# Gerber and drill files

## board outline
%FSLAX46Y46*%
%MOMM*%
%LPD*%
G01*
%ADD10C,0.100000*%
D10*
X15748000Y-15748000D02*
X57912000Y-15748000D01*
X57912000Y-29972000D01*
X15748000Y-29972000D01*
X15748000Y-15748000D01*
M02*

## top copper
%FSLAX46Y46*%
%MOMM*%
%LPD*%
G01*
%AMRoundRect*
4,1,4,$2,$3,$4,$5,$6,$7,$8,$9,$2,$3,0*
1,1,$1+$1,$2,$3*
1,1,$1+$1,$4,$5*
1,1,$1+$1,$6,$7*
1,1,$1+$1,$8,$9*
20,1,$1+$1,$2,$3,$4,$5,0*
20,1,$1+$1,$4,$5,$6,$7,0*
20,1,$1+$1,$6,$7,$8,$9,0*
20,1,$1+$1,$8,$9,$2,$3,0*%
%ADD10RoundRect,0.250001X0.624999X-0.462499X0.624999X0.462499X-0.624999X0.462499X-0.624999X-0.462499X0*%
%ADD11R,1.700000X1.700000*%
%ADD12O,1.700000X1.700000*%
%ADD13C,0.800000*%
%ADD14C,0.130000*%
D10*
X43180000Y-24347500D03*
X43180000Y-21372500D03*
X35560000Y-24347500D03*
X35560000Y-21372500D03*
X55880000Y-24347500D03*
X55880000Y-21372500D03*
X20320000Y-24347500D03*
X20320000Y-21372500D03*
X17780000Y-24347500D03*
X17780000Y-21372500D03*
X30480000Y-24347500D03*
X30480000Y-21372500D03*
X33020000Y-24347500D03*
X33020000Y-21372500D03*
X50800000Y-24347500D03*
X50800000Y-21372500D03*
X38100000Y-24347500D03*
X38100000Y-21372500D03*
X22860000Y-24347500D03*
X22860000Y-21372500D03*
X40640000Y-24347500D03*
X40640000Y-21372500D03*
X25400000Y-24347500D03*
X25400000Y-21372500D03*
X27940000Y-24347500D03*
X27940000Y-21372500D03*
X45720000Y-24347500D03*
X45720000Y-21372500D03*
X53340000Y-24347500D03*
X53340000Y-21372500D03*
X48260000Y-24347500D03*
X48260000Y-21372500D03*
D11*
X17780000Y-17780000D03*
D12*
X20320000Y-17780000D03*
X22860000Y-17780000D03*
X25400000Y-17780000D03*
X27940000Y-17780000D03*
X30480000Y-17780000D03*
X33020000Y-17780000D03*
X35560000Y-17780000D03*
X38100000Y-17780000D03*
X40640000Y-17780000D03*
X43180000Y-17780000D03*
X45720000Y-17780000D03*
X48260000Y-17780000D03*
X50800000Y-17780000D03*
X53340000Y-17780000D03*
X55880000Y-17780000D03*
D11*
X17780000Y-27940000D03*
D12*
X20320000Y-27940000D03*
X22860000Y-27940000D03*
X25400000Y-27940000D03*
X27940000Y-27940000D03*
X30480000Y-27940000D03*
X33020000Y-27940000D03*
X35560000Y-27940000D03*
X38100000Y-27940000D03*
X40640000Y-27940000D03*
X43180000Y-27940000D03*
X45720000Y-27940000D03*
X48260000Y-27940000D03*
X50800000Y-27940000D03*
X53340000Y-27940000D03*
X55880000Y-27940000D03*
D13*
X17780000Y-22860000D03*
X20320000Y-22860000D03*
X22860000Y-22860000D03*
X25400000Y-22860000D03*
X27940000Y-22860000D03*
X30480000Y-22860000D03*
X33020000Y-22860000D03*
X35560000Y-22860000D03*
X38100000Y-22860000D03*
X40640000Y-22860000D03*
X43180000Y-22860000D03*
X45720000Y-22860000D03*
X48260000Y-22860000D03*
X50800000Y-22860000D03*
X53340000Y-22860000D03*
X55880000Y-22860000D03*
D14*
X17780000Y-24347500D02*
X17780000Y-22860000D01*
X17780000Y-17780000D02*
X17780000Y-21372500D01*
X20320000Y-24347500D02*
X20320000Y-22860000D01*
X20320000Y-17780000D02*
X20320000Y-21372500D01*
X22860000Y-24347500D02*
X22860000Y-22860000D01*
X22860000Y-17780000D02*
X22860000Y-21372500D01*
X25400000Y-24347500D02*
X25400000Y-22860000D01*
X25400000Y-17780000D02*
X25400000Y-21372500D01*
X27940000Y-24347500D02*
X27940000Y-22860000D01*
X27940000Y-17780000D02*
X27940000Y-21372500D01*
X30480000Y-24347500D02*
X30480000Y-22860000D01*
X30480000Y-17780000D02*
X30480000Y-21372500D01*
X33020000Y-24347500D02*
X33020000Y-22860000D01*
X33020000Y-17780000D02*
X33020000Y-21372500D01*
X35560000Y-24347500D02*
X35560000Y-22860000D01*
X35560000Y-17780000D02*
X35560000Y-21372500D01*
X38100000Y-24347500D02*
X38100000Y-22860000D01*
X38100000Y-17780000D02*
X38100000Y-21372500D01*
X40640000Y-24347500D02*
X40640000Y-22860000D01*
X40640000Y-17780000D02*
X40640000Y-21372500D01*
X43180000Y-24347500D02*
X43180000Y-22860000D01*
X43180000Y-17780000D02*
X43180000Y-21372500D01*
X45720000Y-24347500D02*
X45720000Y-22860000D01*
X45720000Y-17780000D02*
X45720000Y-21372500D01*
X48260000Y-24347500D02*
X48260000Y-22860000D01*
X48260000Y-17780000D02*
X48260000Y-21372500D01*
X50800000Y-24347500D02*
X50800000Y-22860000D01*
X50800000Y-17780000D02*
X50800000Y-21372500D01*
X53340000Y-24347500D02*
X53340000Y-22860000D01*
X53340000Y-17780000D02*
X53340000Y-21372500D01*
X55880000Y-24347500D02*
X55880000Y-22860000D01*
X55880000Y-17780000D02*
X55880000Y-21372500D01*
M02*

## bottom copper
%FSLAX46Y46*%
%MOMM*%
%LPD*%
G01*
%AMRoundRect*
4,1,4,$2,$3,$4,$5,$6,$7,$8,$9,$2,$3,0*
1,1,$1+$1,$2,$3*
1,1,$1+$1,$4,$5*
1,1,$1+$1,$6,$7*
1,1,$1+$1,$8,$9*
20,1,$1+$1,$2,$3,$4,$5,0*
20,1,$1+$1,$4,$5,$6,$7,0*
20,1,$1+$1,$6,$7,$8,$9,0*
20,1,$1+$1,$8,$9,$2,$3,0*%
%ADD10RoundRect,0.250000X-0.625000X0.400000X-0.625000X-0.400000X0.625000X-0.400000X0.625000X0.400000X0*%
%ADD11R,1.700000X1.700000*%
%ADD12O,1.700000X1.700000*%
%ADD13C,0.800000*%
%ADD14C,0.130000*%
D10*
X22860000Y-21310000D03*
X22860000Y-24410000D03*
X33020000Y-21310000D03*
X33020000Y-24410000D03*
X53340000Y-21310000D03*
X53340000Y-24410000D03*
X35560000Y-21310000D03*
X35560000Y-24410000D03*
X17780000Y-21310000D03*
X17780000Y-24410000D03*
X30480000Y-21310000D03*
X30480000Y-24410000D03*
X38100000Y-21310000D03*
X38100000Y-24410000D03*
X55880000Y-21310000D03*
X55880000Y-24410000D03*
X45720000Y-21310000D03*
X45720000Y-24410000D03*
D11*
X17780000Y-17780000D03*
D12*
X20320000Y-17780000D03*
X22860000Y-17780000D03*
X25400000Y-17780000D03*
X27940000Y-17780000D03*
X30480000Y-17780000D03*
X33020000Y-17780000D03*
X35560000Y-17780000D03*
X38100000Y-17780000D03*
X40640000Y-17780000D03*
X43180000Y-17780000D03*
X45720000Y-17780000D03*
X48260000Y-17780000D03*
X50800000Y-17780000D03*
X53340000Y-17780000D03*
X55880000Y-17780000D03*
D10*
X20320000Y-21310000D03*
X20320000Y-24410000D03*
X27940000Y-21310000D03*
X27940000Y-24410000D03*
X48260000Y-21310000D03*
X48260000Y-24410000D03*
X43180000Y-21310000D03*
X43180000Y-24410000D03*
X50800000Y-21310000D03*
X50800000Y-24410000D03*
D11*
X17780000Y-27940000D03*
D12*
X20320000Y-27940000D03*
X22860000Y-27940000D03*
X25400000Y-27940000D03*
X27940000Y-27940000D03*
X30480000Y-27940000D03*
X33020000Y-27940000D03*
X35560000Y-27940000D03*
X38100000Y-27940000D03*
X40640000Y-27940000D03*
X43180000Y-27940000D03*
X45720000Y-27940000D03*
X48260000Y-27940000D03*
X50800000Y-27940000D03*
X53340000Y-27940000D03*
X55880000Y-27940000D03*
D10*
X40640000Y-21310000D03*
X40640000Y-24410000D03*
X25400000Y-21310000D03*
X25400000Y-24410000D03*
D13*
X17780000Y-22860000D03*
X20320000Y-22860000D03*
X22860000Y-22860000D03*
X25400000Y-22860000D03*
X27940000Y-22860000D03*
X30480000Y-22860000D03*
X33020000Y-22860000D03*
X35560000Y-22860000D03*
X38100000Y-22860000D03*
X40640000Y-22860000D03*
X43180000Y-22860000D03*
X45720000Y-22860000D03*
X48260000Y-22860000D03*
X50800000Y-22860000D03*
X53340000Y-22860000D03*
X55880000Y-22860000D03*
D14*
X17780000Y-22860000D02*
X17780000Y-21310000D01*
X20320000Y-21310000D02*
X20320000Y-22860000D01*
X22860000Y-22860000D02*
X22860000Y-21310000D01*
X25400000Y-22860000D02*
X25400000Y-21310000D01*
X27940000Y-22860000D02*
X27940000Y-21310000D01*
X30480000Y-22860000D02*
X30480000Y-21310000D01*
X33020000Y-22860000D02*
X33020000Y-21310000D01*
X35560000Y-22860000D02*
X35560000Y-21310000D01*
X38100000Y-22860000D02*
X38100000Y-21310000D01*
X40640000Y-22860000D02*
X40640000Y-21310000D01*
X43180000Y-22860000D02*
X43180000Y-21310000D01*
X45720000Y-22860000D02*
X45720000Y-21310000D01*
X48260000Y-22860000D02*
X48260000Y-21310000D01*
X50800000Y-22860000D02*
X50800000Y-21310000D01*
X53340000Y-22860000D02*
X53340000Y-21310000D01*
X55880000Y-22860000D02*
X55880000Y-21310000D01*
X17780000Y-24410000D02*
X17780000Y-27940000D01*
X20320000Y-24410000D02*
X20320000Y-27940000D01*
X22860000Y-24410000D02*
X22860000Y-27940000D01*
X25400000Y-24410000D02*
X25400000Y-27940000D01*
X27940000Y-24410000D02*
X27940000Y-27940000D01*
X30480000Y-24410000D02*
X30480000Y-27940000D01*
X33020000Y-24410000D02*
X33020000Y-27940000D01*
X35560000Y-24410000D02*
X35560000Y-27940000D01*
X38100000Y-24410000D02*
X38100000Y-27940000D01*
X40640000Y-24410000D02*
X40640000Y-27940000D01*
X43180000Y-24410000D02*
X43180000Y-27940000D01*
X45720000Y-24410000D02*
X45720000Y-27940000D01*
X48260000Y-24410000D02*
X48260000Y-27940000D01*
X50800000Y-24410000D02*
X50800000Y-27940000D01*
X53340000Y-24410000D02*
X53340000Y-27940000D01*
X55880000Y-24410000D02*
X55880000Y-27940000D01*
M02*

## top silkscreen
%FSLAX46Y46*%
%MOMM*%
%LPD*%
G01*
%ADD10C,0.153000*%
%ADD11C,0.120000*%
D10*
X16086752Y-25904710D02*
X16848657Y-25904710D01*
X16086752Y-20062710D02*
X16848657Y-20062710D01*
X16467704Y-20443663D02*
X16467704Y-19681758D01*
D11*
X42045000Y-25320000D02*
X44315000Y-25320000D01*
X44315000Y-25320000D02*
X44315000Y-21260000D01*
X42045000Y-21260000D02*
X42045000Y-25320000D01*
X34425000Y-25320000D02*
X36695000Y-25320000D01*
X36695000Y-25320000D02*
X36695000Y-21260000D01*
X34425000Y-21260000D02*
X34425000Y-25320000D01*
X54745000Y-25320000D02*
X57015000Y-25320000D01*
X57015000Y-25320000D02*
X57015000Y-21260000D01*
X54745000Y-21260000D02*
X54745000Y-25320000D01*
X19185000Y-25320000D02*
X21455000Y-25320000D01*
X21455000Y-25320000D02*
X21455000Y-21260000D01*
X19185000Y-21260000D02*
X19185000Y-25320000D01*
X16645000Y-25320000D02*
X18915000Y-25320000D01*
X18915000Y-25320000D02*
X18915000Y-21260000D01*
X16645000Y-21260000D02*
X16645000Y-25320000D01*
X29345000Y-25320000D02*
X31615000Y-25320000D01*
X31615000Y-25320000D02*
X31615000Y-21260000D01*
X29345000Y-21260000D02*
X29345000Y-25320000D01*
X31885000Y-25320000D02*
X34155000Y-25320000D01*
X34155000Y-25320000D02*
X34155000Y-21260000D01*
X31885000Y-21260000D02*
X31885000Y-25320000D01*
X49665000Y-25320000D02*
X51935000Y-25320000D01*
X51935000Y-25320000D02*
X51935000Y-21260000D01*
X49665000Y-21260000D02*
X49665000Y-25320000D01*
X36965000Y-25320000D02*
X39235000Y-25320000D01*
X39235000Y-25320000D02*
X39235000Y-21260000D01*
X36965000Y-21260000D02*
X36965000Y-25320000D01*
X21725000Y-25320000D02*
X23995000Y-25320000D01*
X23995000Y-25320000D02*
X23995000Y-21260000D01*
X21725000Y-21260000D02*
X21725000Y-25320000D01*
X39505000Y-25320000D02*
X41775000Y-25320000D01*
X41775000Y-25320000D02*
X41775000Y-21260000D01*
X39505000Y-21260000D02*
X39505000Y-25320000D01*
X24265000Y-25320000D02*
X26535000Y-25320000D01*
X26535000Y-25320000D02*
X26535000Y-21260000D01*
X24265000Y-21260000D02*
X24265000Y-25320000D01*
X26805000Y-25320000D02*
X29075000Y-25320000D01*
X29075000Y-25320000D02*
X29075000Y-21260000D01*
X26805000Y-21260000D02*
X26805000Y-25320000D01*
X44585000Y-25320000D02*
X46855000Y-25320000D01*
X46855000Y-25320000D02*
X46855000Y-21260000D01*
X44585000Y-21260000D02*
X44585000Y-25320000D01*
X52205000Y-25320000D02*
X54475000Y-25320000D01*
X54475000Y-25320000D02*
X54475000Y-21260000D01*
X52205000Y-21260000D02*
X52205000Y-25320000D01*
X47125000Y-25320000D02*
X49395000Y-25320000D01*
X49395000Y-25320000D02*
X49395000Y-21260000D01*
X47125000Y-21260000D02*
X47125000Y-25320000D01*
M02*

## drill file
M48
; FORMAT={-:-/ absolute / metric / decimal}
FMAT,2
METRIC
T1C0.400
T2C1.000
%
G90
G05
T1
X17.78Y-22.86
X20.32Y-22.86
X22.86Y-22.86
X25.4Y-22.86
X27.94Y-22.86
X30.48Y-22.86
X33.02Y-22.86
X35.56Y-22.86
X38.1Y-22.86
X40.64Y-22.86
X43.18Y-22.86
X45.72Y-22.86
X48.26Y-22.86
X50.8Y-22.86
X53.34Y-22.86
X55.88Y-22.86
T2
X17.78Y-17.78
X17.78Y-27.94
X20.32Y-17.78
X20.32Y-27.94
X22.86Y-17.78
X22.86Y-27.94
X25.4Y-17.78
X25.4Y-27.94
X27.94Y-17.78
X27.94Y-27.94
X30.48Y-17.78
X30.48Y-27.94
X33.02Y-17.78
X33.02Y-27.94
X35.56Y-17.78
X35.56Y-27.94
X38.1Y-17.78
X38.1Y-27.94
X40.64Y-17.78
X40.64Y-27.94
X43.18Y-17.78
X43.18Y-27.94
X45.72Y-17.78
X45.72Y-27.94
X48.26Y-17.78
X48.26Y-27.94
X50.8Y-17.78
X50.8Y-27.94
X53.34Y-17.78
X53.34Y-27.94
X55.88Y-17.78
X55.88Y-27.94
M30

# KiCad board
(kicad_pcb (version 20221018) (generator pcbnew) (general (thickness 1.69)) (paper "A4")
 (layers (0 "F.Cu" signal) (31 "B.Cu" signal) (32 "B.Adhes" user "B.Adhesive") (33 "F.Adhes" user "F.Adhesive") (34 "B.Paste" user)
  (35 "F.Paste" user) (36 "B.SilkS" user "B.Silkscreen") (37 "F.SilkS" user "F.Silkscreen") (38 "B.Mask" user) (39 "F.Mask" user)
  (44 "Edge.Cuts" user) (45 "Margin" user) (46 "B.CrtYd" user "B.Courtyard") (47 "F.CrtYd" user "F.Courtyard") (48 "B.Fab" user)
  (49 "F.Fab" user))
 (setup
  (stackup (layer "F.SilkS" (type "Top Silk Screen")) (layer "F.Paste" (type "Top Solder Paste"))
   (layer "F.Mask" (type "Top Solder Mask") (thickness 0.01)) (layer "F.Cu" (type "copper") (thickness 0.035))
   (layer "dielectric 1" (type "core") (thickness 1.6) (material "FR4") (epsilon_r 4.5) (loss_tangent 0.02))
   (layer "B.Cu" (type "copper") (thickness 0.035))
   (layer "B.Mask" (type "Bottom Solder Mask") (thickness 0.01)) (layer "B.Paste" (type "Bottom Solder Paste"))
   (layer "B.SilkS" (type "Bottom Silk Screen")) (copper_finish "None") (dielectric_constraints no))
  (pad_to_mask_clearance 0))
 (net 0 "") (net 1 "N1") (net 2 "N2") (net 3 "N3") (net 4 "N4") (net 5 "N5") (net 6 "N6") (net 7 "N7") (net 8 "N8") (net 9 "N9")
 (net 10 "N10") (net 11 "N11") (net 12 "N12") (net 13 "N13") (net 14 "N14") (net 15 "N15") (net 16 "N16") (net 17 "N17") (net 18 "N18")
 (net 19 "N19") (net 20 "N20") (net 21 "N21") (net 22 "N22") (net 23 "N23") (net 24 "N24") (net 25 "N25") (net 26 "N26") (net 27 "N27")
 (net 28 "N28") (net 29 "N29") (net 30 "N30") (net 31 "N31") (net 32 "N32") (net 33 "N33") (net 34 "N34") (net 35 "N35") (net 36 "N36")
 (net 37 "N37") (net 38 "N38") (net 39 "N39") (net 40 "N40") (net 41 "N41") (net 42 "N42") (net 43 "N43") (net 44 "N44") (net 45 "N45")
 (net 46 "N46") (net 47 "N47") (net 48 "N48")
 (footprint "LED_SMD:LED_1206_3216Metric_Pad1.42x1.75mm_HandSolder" (layer "F.Cu") (at 43.18 22.86 90)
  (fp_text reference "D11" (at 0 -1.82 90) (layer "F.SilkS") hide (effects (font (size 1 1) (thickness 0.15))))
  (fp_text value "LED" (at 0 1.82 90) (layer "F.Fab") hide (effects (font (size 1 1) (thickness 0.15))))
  (fp_line (start -2.46 -1.135) (end -2.46 1.135) (stroke (width 0.12) (type solid)) (layer "F.SilkS"))
  (fp_line (start -2.46 1.135) (end 1.6 1.135) (stroke (width 0.12) (type solid)) (layer "F.SilkS"))
  (fp_line (start 1.6 -1.135) (end -2.46 -1.135) (stroke (width 0.12) (type solid)) (layer "F.SilkS"))
  (pad "1" smd roundrect (at -1.4875 0 90) (size 1.425 1.75) (layers "F.Cu" "F.Paste" "F.Mask") (roundrect_rratio 0.1754392982) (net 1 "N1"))
  (pad "2" smd roundrect (at 1.4875 0 90) (size 1.425 1.75) (layers "F.Cu" "F.Paste" "F.Mask") (roundrect_rratio 0.1754392982) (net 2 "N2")))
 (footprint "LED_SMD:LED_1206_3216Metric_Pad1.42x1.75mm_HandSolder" (layer "F.Cu") (at 35.56 22.86 90)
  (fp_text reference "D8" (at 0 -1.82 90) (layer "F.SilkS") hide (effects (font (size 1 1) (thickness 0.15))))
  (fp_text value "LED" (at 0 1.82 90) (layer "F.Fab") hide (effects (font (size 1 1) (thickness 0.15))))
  (fp_line (start -2.46 -1.135) (end -2.46 1.135) (stroke (width 0.12) (type solid)) (layer "F.SilkS"))
  (fp_line (start -2.46 1.135) (end 1.6 1.135) (stroke (width 0.12) (type solid)) (layer "F.SilkS"))
  (fp_line (start 1.6 -1.135) (end -2.46 -1.135) (stroke (width 0.12) (type solid)) (layer "F.SilkS"))
  (pad "1" smd roundrect (at -1.4875 0 90) (size 1.425 1.75) (layers "F.Cu" "F.Paste" "F.Mask") (roundrect_rratio 0.1754392982) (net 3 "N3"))
  (pad "2" smd roundrect (at 1.4875 0 90) (size 1.425 1.75) (layers "F.Cu" "F.Paste" "F.Mask") (roundrect_rratio 0.1754392982) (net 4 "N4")))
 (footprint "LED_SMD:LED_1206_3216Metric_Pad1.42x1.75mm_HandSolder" (layer "F.Cu") (at 55.88 22.86 90)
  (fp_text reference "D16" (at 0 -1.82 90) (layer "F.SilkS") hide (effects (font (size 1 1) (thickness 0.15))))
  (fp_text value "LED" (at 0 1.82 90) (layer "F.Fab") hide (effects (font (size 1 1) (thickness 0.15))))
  (fp_line (start -2.46 -1.135) (end -2.46 1.135) (stroke (width 0.12) (type solid)) (layer "F.SilkS"))
  (fp_line (start -2.46 1.135) (end 1.6 1.135) (stroke (width 0.12) (type solid)) (layer "F.SilkS"))
  (fp_line (start 1.6 -1.135) (end -2.46 -1.135) (stroke (width 0.12) (type solid)) (layer "F.SilkS"))
  (pad "1" smd roundrect (at -1.4875 0 90) (size 1.425 1.75) (layers "F.Cu" "F.Paste" "F.Mask") (roundrect_rratio 0.1754392982) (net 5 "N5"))
  (pad "2" smd roundrect (at 1.4875 0 90) (size 1.425 1.75) (layers "F.Cu" "F.Paste" "F.Mask") (roundrect_rratio 0.1754392982) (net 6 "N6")))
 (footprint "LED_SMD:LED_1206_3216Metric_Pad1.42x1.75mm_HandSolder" (layer "F.Cu") (at 20.32 22.86 90)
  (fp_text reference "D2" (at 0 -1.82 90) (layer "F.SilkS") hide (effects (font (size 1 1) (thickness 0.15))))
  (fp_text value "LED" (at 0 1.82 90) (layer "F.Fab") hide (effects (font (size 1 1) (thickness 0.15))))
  (fp_line (start -2.46 -1.135) (end -2.46 1.135) (stroke (width 0.12) (type solid)) (layer "F.SilkS"))
  (fp_line (start -2.46 1.135) (end 1.6 1.135) (stroke (width 0.12) (type solid)) (layer "F.SilkS"))
  (fp_line (start 1.6 -1.135) (end -2.46 -1.135) (stroke (width 0.12) (type solid)) (layer "F.SilkS"))
  (pad "1" smd roundrect (at -1.4875 0 90) (size 1.425 1.75) (layers "F.Cu" "F.Paste" "F.Mask") (roundrect_rratio 0.1754392982) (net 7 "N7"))
  (pad "2" smd roundrect (at 1.4875 0 90) (size 1.425 1.75) (layers "F.Cu" "F.Paste" "F.Mask") (roundrect_rratio 0.1754392982) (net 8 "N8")))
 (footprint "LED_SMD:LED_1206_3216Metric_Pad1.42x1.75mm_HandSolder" (layer "F.Cu") (at 17.78 22.86 90)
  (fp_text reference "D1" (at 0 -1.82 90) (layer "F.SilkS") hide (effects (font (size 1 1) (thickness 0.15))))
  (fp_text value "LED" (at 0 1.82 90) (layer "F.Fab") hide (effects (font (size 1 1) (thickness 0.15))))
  (fp_line (start -2.46 -1.135) (end -2.46 1.135) (stroke (width 0.12) (type solid)) (layer "F.SilkS"))
  (fp_line (start -2.46 1.135) (end 1.6 1.135) (stroke (width 0.12) (type solid)) (layer "F.SilkS"))
  (fp_line (start 1.6 -1.135) (end -2.46 -1.135) (stroke (width 0.12) (type solid)) (layer "F.SilkS"))
  (pad "1" smd roundrect (at -1.4875 0 90) (size 1.425 1.75) (layers "F.Cu" "F.Paste" "F.Mask") (roundrect_rratio 0.1754392982) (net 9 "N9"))
  (pad "2" smd roundrect (at 1.4875 0 90) (size 1.425 1.75) (layers "F.Cu" "F.Paste" "F.Mask") (roundrect_rratio 0.1754392982)
   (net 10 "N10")))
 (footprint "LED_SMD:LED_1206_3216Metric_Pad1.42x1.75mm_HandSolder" (layer "F.Cu") (at 30.48 22.86 90)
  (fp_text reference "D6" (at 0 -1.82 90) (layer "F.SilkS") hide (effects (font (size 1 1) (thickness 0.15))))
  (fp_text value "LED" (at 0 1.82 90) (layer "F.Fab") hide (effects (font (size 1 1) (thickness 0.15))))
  (fp_line (start -2.46 -1.135) (end -2.46 1.135) (stroke (width 0.12) (type solid)) (layer "F.SilkS"))
  (fp_line (start -2.46 1.135) (end 1.6 1.135) (stroke (width 0.12) (type solid)) (layer "F.SilkS"))
  (fp_line (start 1.6 -1.135) (end -2.46 -1.135) (stroke (width 0.12) (type solid)) (layer "F.SilkS"))
  (pad "1" smd roundrect (at -1.4875 0 90) (size 1.425 1.75) (layers "F.Cu" "F.Paste" "F.Mask") (roundrect_rratio 0.1754392982)
   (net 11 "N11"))
  (pad "2" smd roundrect (at 1.4875 0 90) (size 1.425 1.75) (layers "F.Cu" "F.Paste" "F.Mask") (roundrect_rratio 0.1754392982)
   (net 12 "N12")))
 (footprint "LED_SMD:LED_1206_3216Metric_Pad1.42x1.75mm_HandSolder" (layer "F.Cu") (at 33.02 22.86 90)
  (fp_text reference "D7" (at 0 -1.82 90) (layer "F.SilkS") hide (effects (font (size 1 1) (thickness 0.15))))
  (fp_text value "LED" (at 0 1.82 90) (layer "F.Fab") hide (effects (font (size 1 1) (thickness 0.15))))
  (fp_line (start -2.46 -1.135) (end -2.46 1.135) (stroke (width 0.12) (type solid)) (layer "F.SilkS"))
  (fp_line (start -2.46 1.135) (end 1.6 1.135) (stroke (width 0.12) (type solid)) (layer "F.SilkS"))
  (fp_line (start 1.6 -1.135) (end -2.46 -1.135) (stroke (width 0.12) (type solid)) (layer "F.SilkS"))
  (pad "1" smd roundrect (at -1.4875 0 90) (size 1.425 1.75) (layers "F.Cu" "F.Paste" "F.Mask") (roundrect_rratio 0.1754392982)
   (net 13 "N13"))
  (pad "2" smd roundrect (at 1.4875 0 90) (size 1.425 1.75) (layers "F.Cu" "F.Paste" "F.Mask") (roundrect_rratio 0.1754392982)
   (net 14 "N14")))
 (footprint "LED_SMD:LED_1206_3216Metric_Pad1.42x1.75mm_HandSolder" (layer "F.Cu") (at 50.8 22.86 90)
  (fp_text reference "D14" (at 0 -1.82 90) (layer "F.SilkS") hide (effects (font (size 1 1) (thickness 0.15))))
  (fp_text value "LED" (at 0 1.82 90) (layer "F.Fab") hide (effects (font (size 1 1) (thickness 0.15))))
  (fp_line (start -2.46 -1.135) (end -2.46 1.135) (stroke (width 0.12) (type solid)) (layer "F.SilkS"))
  (fp_line (start -2.46 1.135) (end 1.6 1.135) (stroke (width 0.12) (type solid)) (layer "F.SilkS"))
  (fp_line (start 1.6 -1.135) (end -2.46 -1.135) (stroke (width 0.12) (type solid)) (layer "F.SilkS"))
  (pad "1" smd roundrect (at -1.4875 0 90) (size 1.425 1.75) (layers "F.Cu" "F.Paste" "F.Mask") (roundrect_rratio 0.1754392982)
   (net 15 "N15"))
  (pad "2" smd roundrect (at 1.4875 0 90) (size 1.425 1.75) (layers "F.Cu" "F.Paste" "F.Mask") (roundrect_rratio 0.1754392982)
   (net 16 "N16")))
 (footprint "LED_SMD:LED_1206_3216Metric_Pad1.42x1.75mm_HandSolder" (layer "F.Cu") (at 38.1 22.86 90)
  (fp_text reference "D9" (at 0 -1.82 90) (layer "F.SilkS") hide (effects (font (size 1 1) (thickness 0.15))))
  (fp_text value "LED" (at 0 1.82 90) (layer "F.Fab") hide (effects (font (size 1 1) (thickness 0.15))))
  (fp_line (start -2.46 -1.135) (end -2.46 1.135) (stroke (width 0.12) (type solid)) (layer "F.SilkS"))
  (fp_line (start -2.46 1.135) (end 1.6 1.135) (stroke (width 0.12) (type solid)) (layer "F.SilkS"))
  (fp_line (start 1.6 -1.135) (end -2.46 -1.135) (stroke (width 0.12) (type solid)) (layer "F.SilkS"))
  (pad "1" smd roundrect (at -1.4875 0 90) (size 1.425 1.75) (layers "F.Cu" "F.Paste" "F.Mask") (roundrect_rratio 0.1754392982)
   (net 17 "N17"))
  (pad "2" smd roundrect (at 1.4875 0 90) (size 1.425 1.75) (layers "F.Cu" "F.Paste" "F.Mask") (roundrect_rratio 0.1754392982)
   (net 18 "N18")))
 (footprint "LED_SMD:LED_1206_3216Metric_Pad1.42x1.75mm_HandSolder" (layer "F.Cu") (at 22.86 22.86 90)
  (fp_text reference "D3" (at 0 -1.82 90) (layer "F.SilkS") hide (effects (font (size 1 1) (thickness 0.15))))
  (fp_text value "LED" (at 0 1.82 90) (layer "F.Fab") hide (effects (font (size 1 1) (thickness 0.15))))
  (fp_line (start -2.46 -1.135) (end -2.46 1.135) (stroke (width 0.12) (type solid)) (layer "F.SilkS"))
  (fp_line (start -2.46 1.135) (end 1.6 1.135) (stroke (width 0.12) (type solid)) (layer "F.SilkS"))
  (fp_line (start 1.6 -1.135) (end -2.46 -1.135) (stroke (width 0.12) (type solid)) (layer "F.SilkS"))
  (pad "1" smd roundrect (at -1.4875 0 90) (size 1.425 1.75) (layers "F.Cu" "F.Paste" "F.Mask") (roundrect_rratio 0.1754392982)
   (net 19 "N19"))
  (pad "2" smd roundrect (at 1.4875 0 90) (size 1.425 1.75) (layers "F.Cu" "F.Paste" "F.Mask") (roundrect_rratio 0.1754392982)
   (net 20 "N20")))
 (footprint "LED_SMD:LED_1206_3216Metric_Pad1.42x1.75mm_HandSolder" (layer "F.Cu") (at 40.64 22.86 90)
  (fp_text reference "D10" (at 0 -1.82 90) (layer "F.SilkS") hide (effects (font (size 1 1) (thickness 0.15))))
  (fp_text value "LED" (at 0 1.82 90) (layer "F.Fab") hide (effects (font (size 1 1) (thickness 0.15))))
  (fp_line (start -2.46 -1.135) (end -2.46 1.135) (stroke (width 0.12) (type solid)) (layer "F.SilkS"))
  (fp_line (start -2.46 1.135) (end 1.6 1.135) (stroke (width 0.12) (type solid)) (layer "F.SilkS"))
  (fp_line (start 1.6 -1.135) (end -2.46 -1.135) (stroke (width 0.12) (type solid)) (layer "F.SilkS"))
  (pad "1" smd roundrect (at -1.4875 0 90) (size 1.425 1.75) (layers "F.Cu" "F.Paste" "F.Mask") (roundrect_rratio 0.1754392982)
   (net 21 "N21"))
  (pad "2" smd roundrect (at 1.4875 0 90) (size 1.425 1.75) (layers "F.Cu" "F.Paste" "F.Mask") (roundrect_rratio 0.1754392982)
   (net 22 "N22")))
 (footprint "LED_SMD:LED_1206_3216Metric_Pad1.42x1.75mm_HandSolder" (layer "F.Cu") (at 25.4 22.86 90)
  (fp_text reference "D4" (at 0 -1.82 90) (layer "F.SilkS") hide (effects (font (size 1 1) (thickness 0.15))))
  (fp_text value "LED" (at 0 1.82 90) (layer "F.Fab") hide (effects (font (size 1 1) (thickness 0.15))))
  (fp_line (start -2.46 -1.135) (end -2.46 1.135) (stroke (width 0.12) (type solid)) (layer "F.SilkS"))
  (fp_line (start -2.46 1.135) (end 1.6 1.135) (stroke (width 0.12) (type solid)) (layer "F.SilkS"))
  (fp_line (start 1.6 -1.135) (end -2.46 -1.135) (stroke (width 0.12) (type solid)) (layer "F.SilkS"))
  (pad "1" smd roundrect (at -1.4875 0 90) (size 1.425 1.75) (layers "F.Cu" "F.Paste" "F.Mask") (roundrect_rratio 0.1754392982)
   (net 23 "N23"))
  (pad "2" smd roundrect (at 1.4875 0 90) (size 1.425 1.75) (layers "F.Cu" "F.Paste" "F.Mask") (roundrect_rratio 0.1754392982)
   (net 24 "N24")))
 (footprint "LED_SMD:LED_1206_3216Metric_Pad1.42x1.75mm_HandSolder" (layer "F.Cu") (at 27.94 22.86 90)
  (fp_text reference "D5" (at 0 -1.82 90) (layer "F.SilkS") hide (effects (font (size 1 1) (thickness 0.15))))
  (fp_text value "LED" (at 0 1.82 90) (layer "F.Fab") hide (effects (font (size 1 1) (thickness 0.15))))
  (fp_line (start -2.46 -1.135) (end -2.46 1.135) (stroke (width 0.12) (type solid)) (layer "F.SilkS"))
  (fp_line (start -2.46 1.135) (end 1.6 1.135) (stroke (width 0.12) (type solid)) (layer "F.SilkS"))
  (fp_line (start 1.6 -1.135) (end -2.46 -1.135) (stroke (width 0.12) (type solid)) (layer "F.SilkS"))
  (pad "1" smd roundrect (at -1.4875 0 90) (size 1.425 1.75) (layers "F.Cu" "F.Paste" "F.Mask") (roundrect_rratio 0.1754392982)
   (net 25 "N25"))
  (pad "2" smd roundrect (at 1.4875 0 90) (size 1.425 1.75) (layers "F.Cu" "F.Paste" "F.Mask") (roundrect_rratio 0.1754392982)
   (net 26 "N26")))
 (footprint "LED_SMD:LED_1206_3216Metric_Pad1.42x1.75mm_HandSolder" (layer "F.Cu") (at 45.72 22.86 90)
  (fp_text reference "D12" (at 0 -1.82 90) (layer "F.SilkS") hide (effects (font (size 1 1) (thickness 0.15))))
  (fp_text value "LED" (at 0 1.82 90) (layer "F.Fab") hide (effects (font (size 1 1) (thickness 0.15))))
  (fp_line (start -2.46 -1.135) (end -2.46 1.135) (stroke (width 0.12) (type solid)) (layer "F.SilkS"))
  (fp_line (start -2.46 1.135) (end 1.6 1.135) (stroke (width 0.12) (type solid)) (layer "F.SilkS"))
  (fp_line (start 1.6 -1.135) (end -2.46 -1.135) (stroke (width 0.12) (type solid)) (layer "F.SilkS"))
  (pad "1" smd roundrect (at -1.4875 0 90) (size 1.425 1.75) (layers "F.Cu" "F.Paste" "F.Mask") (roundrect_rratio 0.1754392982)
   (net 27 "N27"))
  (pad "2" smd roundrect (at 1.4875 0 90) (size 1.425 1.75) (layers "F.Cu" "F.Paste" "F.Mask") (roundrect_rratio 0.1754392982)
   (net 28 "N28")))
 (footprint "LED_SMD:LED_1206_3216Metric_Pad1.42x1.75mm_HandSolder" (layer "F.Cu") (at 53.34 22.86 90)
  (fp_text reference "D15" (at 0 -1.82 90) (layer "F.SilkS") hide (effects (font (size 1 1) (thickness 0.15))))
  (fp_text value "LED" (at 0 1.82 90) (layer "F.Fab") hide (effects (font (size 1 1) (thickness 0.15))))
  (fp_line (start -2.46 -1.135) (end -2.46 1.135) (stroke (width 0.12) (type solid)) (layer "F.SilkS"))
  (fp_line (start -2.46 1.135) (end 1.6 1.135) (stroke (width 0.12) (type solid)) (layer "F.SilkS"))
  (fp_line (start 1.6 -1.135) (end -2.46 -1.135) (stroke (width 0.12) (type solid)) (layer "F.SilkS"))
  (pad "1" smd roundrect (at -1.4875 0 90) (size 1.425 1.75) (layers "F.Cu" "F.Paste" "F.Mask") (roundrect_rratio 0.1754392982)
   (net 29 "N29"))
  (pad "2" smd roundrect (at 1.4875 0 90) (size 1.425 1.75) (layers "F.Cu" "F.Paste" "F.Mask") (roundrect_rratio 0.1754392982)
   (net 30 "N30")))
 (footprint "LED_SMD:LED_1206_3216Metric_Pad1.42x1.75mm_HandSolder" (layer "F.Cu") (at 48.26 22.86 90)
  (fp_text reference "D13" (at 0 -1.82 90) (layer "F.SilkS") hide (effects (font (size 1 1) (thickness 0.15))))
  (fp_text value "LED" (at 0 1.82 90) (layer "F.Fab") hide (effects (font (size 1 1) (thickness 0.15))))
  (fp_line (start -2.46 -1.135) (end -2.46 1.135) (stroke (width 0.12) (type solid)) (layer "F.SilkS"))
  (fp_line (start -2.46 1.135) (end 1.6 1.135) (stroke (width 0.12) (type solid)) (layer "F.SilkS"))
  (fp_line (start 1.6 -1.135) (end -2.46 -1.135) (stroke (width 0.12) (type solid)) (layer "F.SilkS"))
  (pad "1" smd roundrect (at -1.4875 0 90) (size 1.425 1.75) (layers "F.Cu" "F.Paste" "F.Mask") (roundrect_rratio 0.1754392982)
   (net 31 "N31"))
  (pad "2" smd roundrect (at 1.4875 0 90) (size 1.425 1.75) (layers "F.Cu" "F.Paste" "F.Mask") (roundrect_rratio 0.1754392982)
   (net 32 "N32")))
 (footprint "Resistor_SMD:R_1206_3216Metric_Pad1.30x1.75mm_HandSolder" (layer "B.Cu") (at 22.86 22.86 -90)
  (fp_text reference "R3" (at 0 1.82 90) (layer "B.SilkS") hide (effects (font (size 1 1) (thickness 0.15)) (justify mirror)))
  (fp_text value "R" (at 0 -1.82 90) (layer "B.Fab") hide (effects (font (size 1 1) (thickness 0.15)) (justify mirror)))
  (pad "1" smd roundrect (at -1.55 0 270) (size 1.3 1.75) (layers "B.Cu" "B.Paste" "B.Mask") (roundrect_rratio 0.1923076923) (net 19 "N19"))
  (pad "2" smd roundrect (at 1.55 0 270) (size 1.3 1.75) (layers "B.Cu" "B.Paste" "B.Mask") (roundrect_rratio 0.1923076923) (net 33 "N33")))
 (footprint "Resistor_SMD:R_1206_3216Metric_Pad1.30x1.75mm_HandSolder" (layer "B.Cu") (at 33.02 22.86 -90)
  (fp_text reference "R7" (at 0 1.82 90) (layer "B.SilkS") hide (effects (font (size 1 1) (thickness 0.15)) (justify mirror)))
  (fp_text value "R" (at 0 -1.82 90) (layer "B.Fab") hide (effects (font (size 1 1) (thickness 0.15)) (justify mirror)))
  (pad "1" smd roundrect (at -1.55 0 270) (size 1.3 1.75) (layers "B.Cu" "B.Paste" "B.Mask") (roundrect_rratio 0.1923076923) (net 13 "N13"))
  (pad "2" smd roundrect (at 1.55 0 270) (size 1.3 1.75) (layers "B.Cu" "B.Paste" "B.Mask") (roundrect_rratio 0.1923076923) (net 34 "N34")))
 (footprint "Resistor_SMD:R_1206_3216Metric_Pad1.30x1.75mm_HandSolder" (layer "B.Cu") (at 53.34 22.86 -90)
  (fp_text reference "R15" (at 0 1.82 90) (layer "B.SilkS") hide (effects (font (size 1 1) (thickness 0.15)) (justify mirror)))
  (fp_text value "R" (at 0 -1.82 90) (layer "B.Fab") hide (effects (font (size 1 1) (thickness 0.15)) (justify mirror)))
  (pad "1" smd roundrect (at -1.55 0 270) (size 1.3 1.75) (layers "B.Cu" "B.Paste" "B.Mask") (roundrect_rratio 0.1923076923) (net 29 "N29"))
  (pad "2" smd roundrect (at 1.55 0 270) (size 1.3 1.75) (layers "B.Cu" "B.Paste" "B.Mask") (roundrect_rratio 0.1923076923) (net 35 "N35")))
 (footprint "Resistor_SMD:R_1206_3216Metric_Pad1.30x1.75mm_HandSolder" (layer "B.Cu") (at 35.56 22.86 -90)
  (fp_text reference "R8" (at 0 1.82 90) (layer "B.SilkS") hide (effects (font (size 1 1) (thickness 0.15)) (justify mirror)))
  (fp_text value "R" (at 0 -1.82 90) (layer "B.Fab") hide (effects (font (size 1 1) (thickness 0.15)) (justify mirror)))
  (pad "1" smd roundrect (at -1.55 0 270) (size 1.3 1.75) (layers "B.Cu" "B.Paste" "B.Mask") (roundrect_rratio 0.1923076923) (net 3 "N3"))
  (pad "2" smd roundrect (at 1.55 0 270) (size 1.3 1.75) (layers "B.Cu" "B.Paste" "B.Mask") (roundrect_rratio 0.1923076923) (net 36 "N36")))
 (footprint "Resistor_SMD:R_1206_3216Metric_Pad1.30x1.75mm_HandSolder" (layer "B.Cu") (at 17.78 22.86 -90)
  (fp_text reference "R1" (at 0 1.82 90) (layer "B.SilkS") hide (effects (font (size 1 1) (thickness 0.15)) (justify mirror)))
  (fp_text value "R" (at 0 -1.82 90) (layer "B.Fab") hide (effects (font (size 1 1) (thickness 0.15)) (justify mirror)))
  (pad "1" smd roundrect (at -1.55 0 270) (size 1.3 1.75) (layers "B.Cu" "B.Paste" "B.Mask") (roundrect_rratio 0.1923076923) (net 9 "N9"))
  (pad "2" smd roundrect (at 1.55 0 270) (size 1.3 1.75) (layers "B.Cu" "B.Paste" "B.Mask") (roundrect_rratio 0.1923076923) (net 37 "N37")))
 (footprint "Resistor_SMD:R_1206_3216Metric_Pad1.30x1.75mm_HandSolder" (layer "B.Cu") (at 30.48 22.86 -90)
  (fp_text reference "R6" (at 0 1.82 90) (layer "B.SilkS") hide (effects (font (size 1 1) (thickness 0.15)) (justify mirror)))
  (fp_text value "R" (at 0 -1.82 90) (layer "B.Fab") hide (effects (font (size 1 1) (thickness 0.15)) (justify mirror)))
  (pad "1" smd roundrect (at -1.55 0 270) (size 1.3 1.75) (layers "B.Cu" "B.Paste" "B.Mask") (roundrect_rratio 0.1923076923) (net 11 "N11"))
  (pad "2" smd roundrect (at 1.55 0 270) (size 1.3 1.75) (layers "B.Cu" "B.Paste" "B.Mask") (roundrect_rratio 0.1923076923) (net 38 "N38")))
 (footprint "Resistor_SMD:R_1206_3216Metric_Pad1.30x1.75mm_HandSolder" (layer "B.Cu") (at 38.1 22.86 -90)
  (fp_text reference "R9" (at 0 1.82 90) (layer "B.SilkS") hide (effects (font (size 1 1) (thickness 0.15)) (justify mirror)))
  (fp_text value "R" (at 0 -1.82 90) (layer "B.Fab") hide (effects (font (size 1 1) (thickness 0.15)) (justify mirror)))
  (pad "1" smd roundrect (at -1.55 0 270) (size 1.3 1.75) (layers "B.Cu" "B.Paste" "B.Mask") (roundrect_rratio 0.1923076923) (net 17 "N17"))
  (pad "2" smd roundrect (at 1.55 0 270) (size 1.3 1.75) (layers "B.Cu" "B.Paste" "B.Mask") (roundrect_rratio 0.1923076923) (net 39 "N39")))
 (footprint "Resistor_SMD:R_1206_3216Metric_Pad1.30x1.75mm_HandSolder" (layer "B.Cu") (at 55.88 22.86 -90)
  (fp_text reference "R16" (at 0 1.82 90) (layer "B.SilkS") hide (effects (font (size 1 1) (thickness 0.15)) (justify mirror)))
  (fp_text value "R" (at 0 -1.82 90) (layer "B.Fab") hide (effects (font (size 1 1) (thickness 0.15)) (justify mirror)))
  (pad "1" smd roundrect (at -1.55 0 270) (size 1.3 1.75) (layers "B.Cu" "B.Paste" "B.Mask") (roundrect_rratio 0.1923076923) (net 5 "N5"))
  (pad "2" smd roundrect (at 1.55 0 270) (size 1.3 1.75) (layers "B.Cu" "B.Paste" "B.Mask") (roundrect_rratio 0.1923076923) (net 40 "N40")))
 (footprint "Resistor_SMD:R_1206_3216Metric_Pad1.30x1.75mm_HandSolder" (layer "B.Cu") (at 45.72 22.86 -90)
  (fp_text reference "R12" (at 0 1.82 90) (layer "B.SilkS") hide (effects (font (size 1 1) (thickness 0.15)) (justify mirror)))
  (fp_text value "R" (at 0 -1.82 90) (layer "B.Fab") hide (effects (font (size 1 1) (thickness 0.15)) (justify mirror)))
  (pad "1" smd roundrect (at -1.55 0 270) (size 1.3 1.75) (layers "B.Cu" "B.Paste" "B.Mask") (roundrect_rratio 0.1923076923) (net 27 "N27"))
  (pad "2" smd roundrect (at 1.55 0 270) (size 1.3 1.75) (layers "B.Cu" "B.Paste" "B.Mask") (roundrect_rratio 0.1923076923) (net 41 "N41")))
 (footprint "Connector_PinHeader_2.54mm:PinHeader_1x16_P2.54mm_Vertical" (layer "B.Cu") (at 17.78 17.78 -90)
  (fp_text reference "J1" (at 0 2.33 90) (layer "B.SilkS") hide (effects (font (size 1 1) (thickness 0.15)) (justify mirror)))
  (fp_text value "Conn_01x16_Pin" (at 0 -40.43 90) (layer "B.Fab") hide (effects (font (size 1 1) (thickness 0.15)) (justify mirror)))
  (pad "1" thru_hole rect (at 0 0 270) (size 1.7 1.7) (drill 1) (layers "*.Cu" "*.Mask") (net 10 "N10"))
  (pad "2" thru_hole oval (at 0 -2.54 270) (size 1.7 1.7) (drill 1) (layers "*.Cu" "*.Mask") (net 8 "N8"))
  (pad "3" thru_hole oval (at 0 -5.08 270) (size 1.7 1.7) (drill 1) (layers "*.Cu" "*.Mask") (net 20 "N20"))
  (pad "4" thru_hole oval (at 0 -7.62 270) (size 1.7 1.7) (drill 1) (layers "*.Cu" "*.Mask") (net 24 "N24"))
  (pad "5" thru_hole oval (at 0 -10.16 270) (size 1.7 1.7) (drill 1) (layers "*.Cu" "*.Mask") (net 26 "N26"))
  (pad "6" thru_hole oval (at 0 -12.7 270) (size 1.7 1.7) (drill 1) (layers "*.Cu" "*.Mask") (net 12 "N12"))
  (pad "7" thru_hole oval (at 0 -15.24 270) (size 1.7 1.7) (drill 1) (layers "*.Cu" "*.Mask") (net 14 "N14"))
  (pad "8" thru_hole oval (at 0 -17.78 270) (size 1.7 1.7) (drill 1) (layers "*.Cu" "*.Mask") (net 4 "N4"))
  (pad "9" thru_hole oval (at 0 -20.32 270) (size 1.7 1.7) (drill 1) (layers "*.Cu" "*.Mask") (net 18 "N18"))
  (pad "10" thru_hole oval (at 0 -22.86 270) (size 1.7 1.7) (drill 1) (layers "*.Cu" "*.Mask") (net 22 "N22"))
  (pad "11" thru_hole oval (at 0 -25.4 270) (size 1.7 1.7) (drill 1) (layers "*.Cu" "*.Mask") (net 2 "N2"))
  (pad "12" thru_hole oval (at 0 -27.94 270) (size 1.7 1.7) (drill 1) (layers "*.Cu" "*.Mask") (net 28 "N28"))
  (pad "13" thru_hole oval (at 0 -30.48 270) (size 1.7 1.7) (drill 1) (layers "*.Cu" "*.Mask") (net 32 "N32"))
  (pad "14" thru_hole oval (at 0 -33.02 270) (size 1.7 1.7) (drill 1) (layers "*.Cu" "*.Mask") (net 16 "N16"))
  (pad "15" thru_hole oval (at 0 -35.56 270) (size 1.7 1.7) (drill 1) (layers "*.Cu" "*.Mask") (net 30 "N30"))
  (pad "16" thru_hole oval (at 0 -38.1 270) (size 1.7 1.7) (drill 1) (layers "*.Cu" "*.Mask") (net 6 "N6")))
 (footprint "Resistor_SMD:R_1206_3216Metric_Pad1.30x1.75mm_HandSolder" (layer "B.Cu") (at 20.32 22.86 -90)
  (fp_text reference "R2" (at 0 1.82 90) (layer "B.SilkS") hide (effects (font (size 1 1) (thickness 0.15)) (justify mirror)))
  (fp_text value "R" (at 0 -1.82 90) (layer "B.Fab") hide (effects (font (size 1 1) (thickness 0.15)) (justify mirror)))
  (pad "1" smd roundrect (at -1.55 0 270) (size 1.3 1.75) (layers "B.Cu" "B.Paste" "B.Mask") (roundrect_rratio 0.1923076923) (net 7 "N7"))
  (pad "2" smd roundrect (at 1.55 0 270) (size 1.3 1.75) (layers "B.Cu" "B.Paste" "B.Mask") (roundrect_rratio 0.1923076923) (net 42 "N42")))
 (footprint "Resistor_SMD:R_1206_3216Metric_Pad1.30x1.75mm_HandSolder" (layer "B.Cu") (at 27.94 22.86 -90)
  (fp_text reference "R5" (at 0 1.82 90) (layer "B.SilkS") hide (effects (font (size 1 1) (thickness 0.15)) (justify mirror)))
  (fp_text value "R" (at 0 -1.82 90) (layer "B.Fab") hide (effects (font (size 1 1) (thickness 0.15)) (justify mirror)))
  (pad "1" smd roundrect (at -1.55 0 270) (size 1.3 1.75) (layers "B.Cu" "B.Paste" "B.Mask") (roundrect_rratio 0.1923076923) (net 25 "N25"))
  (pad "2" smd roundrect (at 1.55 0 270) (size 1.3 1.75) (layers "B.Cu" "B.Paste" "B.Mask") (roundrect_rratio 0.1923076923) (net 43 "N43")))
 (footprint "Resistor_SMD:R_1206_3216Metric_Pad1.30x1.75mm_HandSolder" (layer "B.Cu") (at 48.26 22.86 -90)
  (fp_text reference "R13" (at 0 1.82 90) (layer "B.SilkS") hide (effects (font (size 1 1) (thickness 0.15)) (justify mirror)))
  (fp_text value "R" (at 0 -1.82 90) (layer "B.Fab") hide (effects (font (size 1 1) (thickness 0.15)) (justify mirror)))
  (pad "1" smd roundrect (at -1.55 0 270) (size 1.3 1.75) (layers "B.Cu" "B.Paste" "B.Mask") (roundrect_rratio 0.1923076923) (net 31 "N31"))
  (pad "2" smd roundrect (at 1.55 0 270) (size 1.3 1.75) (layers "B.Cu" "B.Paste" "B.Mask") (roundrect_rratio 0.1923076923) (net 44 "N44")))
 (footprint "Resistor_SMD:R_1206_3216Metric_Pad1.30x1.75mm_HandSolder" (layer "B.Cu") (at 43.18 22.86 -90)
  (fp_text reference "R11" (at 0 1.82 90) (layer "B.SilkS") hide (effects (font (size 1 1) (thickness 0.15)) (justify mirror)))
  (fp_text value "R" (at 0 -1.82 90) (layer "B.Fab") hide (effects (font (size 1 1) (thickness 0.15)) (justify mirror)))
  (pad "1" smd roundrect (at -1.55 0 270) (size 1.3 1.75) (layers "B.Cu" "B.Paste" "B.Mask") (roundrect_rratio 0.1923076923) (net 1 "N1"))
  (pad "2" smd roundrect (at 1.55 0 270) (size 1.3 1.75) (layers "B.Cu" "B.Paste" "B.Mask") (roundrect_rratio 0.1923076923) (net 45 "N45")))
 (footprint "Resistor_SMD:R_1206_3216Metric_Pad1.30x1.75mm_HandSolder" (layer "B.Cu") (at 50.8 22.86 -90)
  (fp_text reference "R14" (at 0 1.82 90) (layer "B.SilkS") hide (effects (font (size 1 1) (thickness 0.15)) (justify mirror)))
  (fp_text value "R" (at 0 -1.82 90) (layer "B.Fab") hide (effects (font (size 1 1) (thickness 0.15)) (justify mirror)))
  (pad "1" smd roundrect (at -1.55 0 270) (size 1.3 1.75) (layers "B.Cu" "B.Paste" "B.Mask") (roundrect_rratio 0.1923076923) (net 15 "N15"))
  (pad "2" smd roundrect (at 1.55 0 270) (size 1.3 1.75) (layers "B.Cu" "B.Paste" "B.Mask") (roundrect_rratio 0.1923076923) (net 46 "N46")))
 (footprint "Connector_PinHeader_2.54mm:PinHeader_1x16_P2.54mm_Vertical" (layer "B.Cu") (at 17.78 27.94 -90)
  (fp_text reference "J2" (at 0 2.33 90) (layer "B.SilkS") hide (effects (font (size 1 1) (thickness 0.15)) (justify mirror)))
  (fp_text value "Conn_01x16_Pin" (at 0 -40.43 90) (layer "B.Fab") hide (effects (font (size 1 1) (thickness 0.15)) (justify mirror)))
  (pad "1" thru_hole rect (at 0 0 270) (size 1.7 1.7) (drill 1) (layers "*.Cu" "*.Mask") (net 37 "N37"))
  (pad "2" thru_hole oval (at 0 -2.54 270) (size 1.7 1.7) (drill 1) (layers "*.Cu" "*.Mask") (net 42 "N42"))
  (pad "3" thru_hole oval (at 0 -5.08 270) (size 1.7 1.7) (drill 1) (layers "*.Cu" "*.Mask") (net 33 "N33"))
  (pad "4" thru_hole oval (at 0 -7.62 270) (size 1.7 1.7) (drill 1) (layers "*.Cu" "*.Mask") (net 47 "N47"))
  (pad "5" thru_hole oval (at 0 -10.16 270) (size 1.7 1.7) (drill 1) (layers "*.Cu" "*.Mask") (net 43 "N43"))
  (pad "6" thru_hole oval (at 0 -12.7 270) (size 1.7 1.7) (drill 1) (layers "*.Cu" "*.Mask") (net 38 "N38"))
  (pad "7" thru_hole oval (at 0 -15.24 270) (size 1.7 1.7) (drill 1) (layers "*.Cu" "*.Mask") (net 34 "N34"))
  (pad "8" thru_hole oval (at 0 -17.78 270) (size 1.7 1.7) (drill 1) (layers "*.Cu" "*.Mask") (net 36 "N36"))
  (pad "9" thru_hole oval (at 0 -20.32 270) (size 1.7 1.7) (drill 1) (layers "*.Cu" "*.Mask") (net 39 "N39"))
  (pad "10" thru_hole oval (at 0 -22.86 270) (size 1.7 1.7) (drill 1) (layers "*.Cu" "*.Mask") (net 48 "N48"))
  (pad "11" thru_hole oval (at 0 -25.4 270) (size 1.7 1.7) (drill 1) (layers "*.Cu" "*.Mask") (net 45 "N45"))
  (pad "12" thru_hole oval (at 0 -27.94 270) (size 1.7 1.7) (drill 1) (layers "*.Cu" "*.Mask") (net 41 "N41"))
  (pad "13" thru_hole oval (at 0 -30.48 270) (size 1.7 1.7) (drill 1) (layers "*.Cu" "*.Mask") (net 44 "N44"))
  (pad "14" thru_hole oval (at 0 -33.02 270) (size 1.7 1.7) (drill 1) (layers "*.Cu" "*.Mask") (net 46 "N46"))
  (pad "15" thru_hole oval (at 0 -35.56 270) (size 1.7 1.7) (drill 1) (layers "*.Cu" "*.Mask") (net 35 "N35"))
  (pad "16" thru_hole oval (at 0 -38.1 270) (size 1.7 1.7) (drill 1) (layers "*.Cu" "*.Mask") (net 40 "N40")))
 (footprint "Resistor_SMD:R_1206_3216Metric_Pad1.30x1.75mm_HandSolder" (layer "B.Cu") (at 40.64 22.86 -90)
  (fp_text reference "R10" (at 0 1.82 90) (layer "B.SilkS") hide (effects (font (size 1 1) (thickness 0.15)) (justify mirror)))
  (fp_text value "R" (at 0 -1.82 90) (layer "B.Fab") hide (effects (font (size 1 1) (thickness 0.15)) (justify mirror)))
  (pad "1" smd roundrect (at -1.55 0 270) (size 1.3 1.75) (layers "B.Cu" "B.Paste" "B.Mask") (roundrect_rratio 0.1923076923) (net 21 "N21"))
  (pad "2" smd roundrect (at 1.55 0 270) (size 1.3 1.75) (layers "B.Cu" "B.Paste" "B.Mask") (roundrect_rratio 0.1923076923) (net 48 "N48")))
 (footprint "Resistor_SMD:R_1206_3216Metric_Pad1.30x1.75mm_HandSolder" (layer "B.Cu") (at 25.4 22.86 -90)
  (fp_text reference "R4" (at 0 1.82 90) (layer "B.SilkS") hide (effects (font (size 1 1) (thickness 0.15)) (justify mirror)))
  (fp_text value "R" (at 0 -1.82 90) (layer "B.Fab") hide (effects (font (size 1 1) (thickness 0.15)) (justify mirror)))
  (pad "1" smd roundrect (at -1.55 0 270) (size 1.3 1.75) (layers "B.Cu" "B.Paste" "B.Mask") (roundrect_rratio 0.1923076923) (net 23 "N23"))
  (pad "2" smd roundrect (at 1.55 0 270) (size 1.3 1.75) (layers "B.Cu" "B.Paste" "B.Mask") (roundrect_rratio 0.1923076923) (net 47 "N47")))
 (gr_rect (start 15.748 15.748) (end 57.912 29.972) (stroke (width 0.1) (type default)) (fill none) (layer "Edge.Cuts"))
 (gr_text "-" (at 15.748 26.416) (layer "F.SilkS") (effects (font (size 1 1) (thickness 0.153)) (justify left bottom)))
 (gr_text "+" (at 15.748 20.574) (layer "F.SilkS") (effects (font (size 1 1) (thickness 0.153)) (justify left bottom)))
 (segment (start 17.78 24.3475) (end 17.78 22.86) (width 0.13) (layer "F.Cu") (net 9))
 (via (at 17.78 22.86) (size 0.8) (drill 0.4) (layers "F.Cu" "B.Cu") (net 9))
 (segment (start 17.78 22.86) (end 17.78 21.31) (width 0.13) (layer "B.Cu") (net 9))
 (segment (start 17.78 17.78) (end 17.78 21.3725) (width 0.13) (layer "F.Cu") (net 10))
 (segment (start 20.32 24.3475) (end 20.32 22.86) (width 0.13) (layer "F.Cu") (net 7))
 (via (at 20.32 22.86) (size 0.8) (drill 0.4) (layers "F.Cu" "B.Cu") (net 7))
 (segment (start 20.32 21.31) (end 20.32 22.86) (width 0.13) (layer "B.Cu") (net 7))
 (segment (start 20.32 17.78) (end 20.32 21.3725) (width 0.13) (layer "F.Cu") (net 8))
 (segment (start 22.86 24.3475) (end 22.86 22.86) (width 0.13) (layer "F.Cu") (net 19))
 (via (at 22.86 22.86) (size 0.8) (drill 0.4) (layers "F.Cu" "B.Cu") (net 19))
 (segment (start 22.86 22.86) (end 22.86 21.31) (width 0.13) (layer "B.Cu") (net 19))
 (segment (start 22.86 17.78) (end 22.86 21.3725) (width 0.13) (layer "F.Cu") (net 20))
 (segment (start 25.4 24.3475) (end 25.4 22.86) (width 0.13) (layer "F.Cu") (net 23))
 (via (at 25.4 22.86) (size 0.8) (drill 0.4) (layers "F.Cu" "B.Cu") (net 23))
 (segment (start 25.4 22.86) (end 25.4 21.31) (width 0.13) (layer "B.Cu") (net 23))
 (segment (start 25.4 17.78) (end 25.4 21.3725) (width 0.13) (layer "F.Cu") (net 24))
 (segment (start 27.94 24.3475) (end 27.94 22.86) (width 0.13) (layer "F.Cu") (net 25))
 (via (at 27.94 22.86) (size 0.8) (drill 0.4) (layers "F.Cu" "B.Cu") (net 25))
 (segment (start 27.94 22.86) (end 27.94 21.31) (width 0.13) (layer "B.Cu") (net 25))
 (segment (start 27.94 17.78) (end 27.94 21.3725) (width 0.13) (layer "F.Cu") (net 26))
 (segment (start 30.48 24.3475) (end 30.48 22.86) (width 0.13) (layer "F.Cu") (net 11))
 (via (at 30.48 22.86) (size 0.8) (drill 0.4) (layers "F.Cu" "B.Cu") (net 11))
 (segment (start 30.48 22.86) (end 30.48 21.31) (width 0.13) (layer "B.Cu") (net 11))
 (segment (start 30.48 17.78) (end 30.48 21.3725) (width 0.13) (layer "F.Cu") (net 12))
 (segment (start 33.02 24.3475) (end 33.02 22.86) (width 0.13) (layer "F.Cu") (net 13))
 (via (at 33.02 22.86) (size 0.8) (drill 0.4) (layers "F.Cu" "B.Cu") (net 13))
 (segment (start 33.02 22.86) (end 33.02 21.31) (width 0.13) (layer "B.Cu") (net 13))
 (segment (start 33.02 17.78) (end 33.02 21.3725) (width 0.13) (layer "F.Cu") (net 14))
 (segment (start 35.56 24.3475) (end 35.56 22.86) (width 0.13) (layer "F.Cu") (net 3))
 (via (at 35.56 22.86) (size 0.8) (drill 0.4) (layers "F.Cu" "B.Cu") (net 3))
 (segment (start 35.56 22.86) (end 35.56 21.31) (width 0.13) (layer "B.Cu") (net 3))
 (segment (start 35.56 17.78) (end 35.56 21.3725) (width 0.13) (layer "F.Cu") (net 4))
 (segment (start 38.1 24.3475) (end 38.1 22.86) (width 0.13) (layer "F.Cu") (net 17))
 (via (at 38.1 22.86) (size 0.8) (drill 0.4) (layers "F.Cu" "B.Cu") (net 17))
 (segment (start 38.1 22.86) (end 38.1 21.31) (width 0.13) (layer "B.Cu") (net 17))
 (segment (start 38.1 17.78) (end 38.1 21.3725) (width 0.13) (layer "F.Cu") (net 18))
 (segment (start 40.64 24.3475) (end 40.64 22.86) (width 0.13) (layer "F.Cu") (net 21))
 (via (at 40.64 22.86) (size 0.8) (drill 0.4) (layers "F.Cu" "B.Cu") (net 21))
 (segment (start 40.64 22.86) (end 40.64 21.31) (width 0.13) (layer "B.Cu") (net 21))
 (segment (start 40.64 17.78) (end 40.64 21.3725) (width 0.13) (layer "F.Cu") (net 22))
 (segment (start 43.18 24.3475) (end 43.18 22.86) (width 0.13) (layer "F.Cu") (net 1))
 (via (at 43.18 22.86) (size 0.8) (drill 0.4) (layers "F.Cu" "B.Cu") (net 1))
 (segment (start 43.18 22.86) (end 43.18 21.31) (width 0.13) (layer "B.Cu") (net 1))
 (segment (start 43.18 17.78) (end 43.18 21.3725) (width 0.13) (layer "F.Cu") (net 2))
 (segment (start 45.72 24.3475) (end 45.72 22.86) (width 0.13) (layer "F.Cu") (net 27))
 (via (at 45.72 22.86) (size 0.8) (drill 0.4) (layers "F.Cu" "B.Cu") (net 27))
 (segment (start 45.72 22.86) (end 45.72 21.31) (width 0.13) (layer "B.Cu") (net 27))
 (segment (start 45.72 17.78) (end 45.72 21.3725) (width 0.13) (layer "F.Cu") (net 28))
 (segment (start 48.26 24.3475) (end 48.26 22.86) (width 0.13) (layer "F.Cu") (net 31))
 (via (at 48.26 22.86) (size 0.8) (drill 0.4) (layers "F.Cu" "B.Cu") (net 31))
 (segment (start 48.26 22.86) (end 48.26 21.31) (width 0.13) (layer "B.Cu") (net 31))
 (segment (start 48.26 17.78) (end 48.26 21.3725) (width 0.13) (layer "F.Cu") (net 32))
 (segment (start 50.8 24.3475) (end 50.8 22.86) (width 0.13) (layer "F.Cu") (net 15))
 (via (at 50.8 22.86) (size 0.8) (drill 0.4) (layers "F.Cu" "B.Cu") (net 15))
 (segment (start 50.8 22.86) (end 50.8 21.31) (width 0.13) (layer "B.Cu") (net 15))
 (segment (start 50.8 17.78) (end 50.8 21.3725) (width 0.13) (layer "F.Cu") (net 16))
 (segment (start 53.34 24.3475) (end 53.34 22.86) (width 0.13) (layer "F.Cu") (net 29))
 (via (at 53.34 22.86) (size 0.8) (drill 0.4) (layers "F.Cu" "B.Cu") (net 29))
 (segment (start 53.34 22.86) (end 53.34 21.31) (width 0.13) (layer "B.Cu") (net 29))
 (segment (start 53.34 17.78) (end 53.34 21.3725) (width 0.13) (layer "F.Cu") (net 30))
 (segment (start 55.88 24.3475) (end 55.88 22.86) (width 0.13) (layer "F.Cu") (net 5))
 (via (at 55.88 22.86) (size 0.8) (drill 0.4) (layers "F.Cu" "B.Cu") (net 5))
 (segment (start 55.88 22.86) (end 55.88 21.31) (width 0.13) (layer "B.Cu") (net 5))
 (segment (start 55.88 17.78) (end 55.88 21.3725) (width 0.13) (layer "F.Cu") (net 6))
 (segment (start 17.78 24.41) (end 17.78 27.94) (width 0.13) (layer "B.Cu") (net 37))
 (segment (start 20.32 24.41) (end 20.32 27.94) (width 0.13) (layer "B.Cu") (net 42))
 (segment (start 22.86 24.41) (end 22.86 27.94) (width 0.13) (layer "B.Cu") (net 33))
 (segment (start 25.4 24.41) (end 25.4 27.94) (width 0.13) (layer "B.Cu") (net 47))
 (segment (start 27.94 24.41) (end 27.94 27.94) (width 0.13) (layer "B.Cu") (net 43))
 (segment (start 30.48 24.41) (end 30.48 27.94) (width 0.13) (layer "B.Cu") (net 38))
 (segment (start 33.02 24.41) (end 33.02 27.94) (width 0.13) (layer "B.Cu") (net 34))
 (segment (start 35.56 24.41) (end 35.56 27.94) (width 0.13) (layer "B.Cu") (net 36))
 (segment (start 38.1 24.41) (end 38.1 27.94) (width 0.13) (layer "B.Cu") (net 39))
 (segment (start 40.64 24.41) (end 40.64 27.94) (width 0.13) (layer "B.Cu") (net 48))
 (segment (start 43.18 24.41) (end 43.18 27.94) (width 0.13) (layer "B.Cu") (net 45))
 (segment (start 45.72 24.41) (end 45.72 27.94) (width 0.13) (layer "B.Cu") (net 41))
 (segment (start 48.26 24.41) (end 48.26 27.94) (width 0.13) (layer "B.Cu") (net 44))
 (segment (start 50.8 24.41) (end 50.8 27.94) (width 0.13) (layer "B.Cu") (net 46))
 (segment (start 53.34 24.41) (end 53.34 27.94) (width 0.13) (layer "B.Cu") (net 35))
 (segment (start 55.88 24.41) (end 55.88 27.94) (width 0.13) (layer "B.Cu") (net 40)))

